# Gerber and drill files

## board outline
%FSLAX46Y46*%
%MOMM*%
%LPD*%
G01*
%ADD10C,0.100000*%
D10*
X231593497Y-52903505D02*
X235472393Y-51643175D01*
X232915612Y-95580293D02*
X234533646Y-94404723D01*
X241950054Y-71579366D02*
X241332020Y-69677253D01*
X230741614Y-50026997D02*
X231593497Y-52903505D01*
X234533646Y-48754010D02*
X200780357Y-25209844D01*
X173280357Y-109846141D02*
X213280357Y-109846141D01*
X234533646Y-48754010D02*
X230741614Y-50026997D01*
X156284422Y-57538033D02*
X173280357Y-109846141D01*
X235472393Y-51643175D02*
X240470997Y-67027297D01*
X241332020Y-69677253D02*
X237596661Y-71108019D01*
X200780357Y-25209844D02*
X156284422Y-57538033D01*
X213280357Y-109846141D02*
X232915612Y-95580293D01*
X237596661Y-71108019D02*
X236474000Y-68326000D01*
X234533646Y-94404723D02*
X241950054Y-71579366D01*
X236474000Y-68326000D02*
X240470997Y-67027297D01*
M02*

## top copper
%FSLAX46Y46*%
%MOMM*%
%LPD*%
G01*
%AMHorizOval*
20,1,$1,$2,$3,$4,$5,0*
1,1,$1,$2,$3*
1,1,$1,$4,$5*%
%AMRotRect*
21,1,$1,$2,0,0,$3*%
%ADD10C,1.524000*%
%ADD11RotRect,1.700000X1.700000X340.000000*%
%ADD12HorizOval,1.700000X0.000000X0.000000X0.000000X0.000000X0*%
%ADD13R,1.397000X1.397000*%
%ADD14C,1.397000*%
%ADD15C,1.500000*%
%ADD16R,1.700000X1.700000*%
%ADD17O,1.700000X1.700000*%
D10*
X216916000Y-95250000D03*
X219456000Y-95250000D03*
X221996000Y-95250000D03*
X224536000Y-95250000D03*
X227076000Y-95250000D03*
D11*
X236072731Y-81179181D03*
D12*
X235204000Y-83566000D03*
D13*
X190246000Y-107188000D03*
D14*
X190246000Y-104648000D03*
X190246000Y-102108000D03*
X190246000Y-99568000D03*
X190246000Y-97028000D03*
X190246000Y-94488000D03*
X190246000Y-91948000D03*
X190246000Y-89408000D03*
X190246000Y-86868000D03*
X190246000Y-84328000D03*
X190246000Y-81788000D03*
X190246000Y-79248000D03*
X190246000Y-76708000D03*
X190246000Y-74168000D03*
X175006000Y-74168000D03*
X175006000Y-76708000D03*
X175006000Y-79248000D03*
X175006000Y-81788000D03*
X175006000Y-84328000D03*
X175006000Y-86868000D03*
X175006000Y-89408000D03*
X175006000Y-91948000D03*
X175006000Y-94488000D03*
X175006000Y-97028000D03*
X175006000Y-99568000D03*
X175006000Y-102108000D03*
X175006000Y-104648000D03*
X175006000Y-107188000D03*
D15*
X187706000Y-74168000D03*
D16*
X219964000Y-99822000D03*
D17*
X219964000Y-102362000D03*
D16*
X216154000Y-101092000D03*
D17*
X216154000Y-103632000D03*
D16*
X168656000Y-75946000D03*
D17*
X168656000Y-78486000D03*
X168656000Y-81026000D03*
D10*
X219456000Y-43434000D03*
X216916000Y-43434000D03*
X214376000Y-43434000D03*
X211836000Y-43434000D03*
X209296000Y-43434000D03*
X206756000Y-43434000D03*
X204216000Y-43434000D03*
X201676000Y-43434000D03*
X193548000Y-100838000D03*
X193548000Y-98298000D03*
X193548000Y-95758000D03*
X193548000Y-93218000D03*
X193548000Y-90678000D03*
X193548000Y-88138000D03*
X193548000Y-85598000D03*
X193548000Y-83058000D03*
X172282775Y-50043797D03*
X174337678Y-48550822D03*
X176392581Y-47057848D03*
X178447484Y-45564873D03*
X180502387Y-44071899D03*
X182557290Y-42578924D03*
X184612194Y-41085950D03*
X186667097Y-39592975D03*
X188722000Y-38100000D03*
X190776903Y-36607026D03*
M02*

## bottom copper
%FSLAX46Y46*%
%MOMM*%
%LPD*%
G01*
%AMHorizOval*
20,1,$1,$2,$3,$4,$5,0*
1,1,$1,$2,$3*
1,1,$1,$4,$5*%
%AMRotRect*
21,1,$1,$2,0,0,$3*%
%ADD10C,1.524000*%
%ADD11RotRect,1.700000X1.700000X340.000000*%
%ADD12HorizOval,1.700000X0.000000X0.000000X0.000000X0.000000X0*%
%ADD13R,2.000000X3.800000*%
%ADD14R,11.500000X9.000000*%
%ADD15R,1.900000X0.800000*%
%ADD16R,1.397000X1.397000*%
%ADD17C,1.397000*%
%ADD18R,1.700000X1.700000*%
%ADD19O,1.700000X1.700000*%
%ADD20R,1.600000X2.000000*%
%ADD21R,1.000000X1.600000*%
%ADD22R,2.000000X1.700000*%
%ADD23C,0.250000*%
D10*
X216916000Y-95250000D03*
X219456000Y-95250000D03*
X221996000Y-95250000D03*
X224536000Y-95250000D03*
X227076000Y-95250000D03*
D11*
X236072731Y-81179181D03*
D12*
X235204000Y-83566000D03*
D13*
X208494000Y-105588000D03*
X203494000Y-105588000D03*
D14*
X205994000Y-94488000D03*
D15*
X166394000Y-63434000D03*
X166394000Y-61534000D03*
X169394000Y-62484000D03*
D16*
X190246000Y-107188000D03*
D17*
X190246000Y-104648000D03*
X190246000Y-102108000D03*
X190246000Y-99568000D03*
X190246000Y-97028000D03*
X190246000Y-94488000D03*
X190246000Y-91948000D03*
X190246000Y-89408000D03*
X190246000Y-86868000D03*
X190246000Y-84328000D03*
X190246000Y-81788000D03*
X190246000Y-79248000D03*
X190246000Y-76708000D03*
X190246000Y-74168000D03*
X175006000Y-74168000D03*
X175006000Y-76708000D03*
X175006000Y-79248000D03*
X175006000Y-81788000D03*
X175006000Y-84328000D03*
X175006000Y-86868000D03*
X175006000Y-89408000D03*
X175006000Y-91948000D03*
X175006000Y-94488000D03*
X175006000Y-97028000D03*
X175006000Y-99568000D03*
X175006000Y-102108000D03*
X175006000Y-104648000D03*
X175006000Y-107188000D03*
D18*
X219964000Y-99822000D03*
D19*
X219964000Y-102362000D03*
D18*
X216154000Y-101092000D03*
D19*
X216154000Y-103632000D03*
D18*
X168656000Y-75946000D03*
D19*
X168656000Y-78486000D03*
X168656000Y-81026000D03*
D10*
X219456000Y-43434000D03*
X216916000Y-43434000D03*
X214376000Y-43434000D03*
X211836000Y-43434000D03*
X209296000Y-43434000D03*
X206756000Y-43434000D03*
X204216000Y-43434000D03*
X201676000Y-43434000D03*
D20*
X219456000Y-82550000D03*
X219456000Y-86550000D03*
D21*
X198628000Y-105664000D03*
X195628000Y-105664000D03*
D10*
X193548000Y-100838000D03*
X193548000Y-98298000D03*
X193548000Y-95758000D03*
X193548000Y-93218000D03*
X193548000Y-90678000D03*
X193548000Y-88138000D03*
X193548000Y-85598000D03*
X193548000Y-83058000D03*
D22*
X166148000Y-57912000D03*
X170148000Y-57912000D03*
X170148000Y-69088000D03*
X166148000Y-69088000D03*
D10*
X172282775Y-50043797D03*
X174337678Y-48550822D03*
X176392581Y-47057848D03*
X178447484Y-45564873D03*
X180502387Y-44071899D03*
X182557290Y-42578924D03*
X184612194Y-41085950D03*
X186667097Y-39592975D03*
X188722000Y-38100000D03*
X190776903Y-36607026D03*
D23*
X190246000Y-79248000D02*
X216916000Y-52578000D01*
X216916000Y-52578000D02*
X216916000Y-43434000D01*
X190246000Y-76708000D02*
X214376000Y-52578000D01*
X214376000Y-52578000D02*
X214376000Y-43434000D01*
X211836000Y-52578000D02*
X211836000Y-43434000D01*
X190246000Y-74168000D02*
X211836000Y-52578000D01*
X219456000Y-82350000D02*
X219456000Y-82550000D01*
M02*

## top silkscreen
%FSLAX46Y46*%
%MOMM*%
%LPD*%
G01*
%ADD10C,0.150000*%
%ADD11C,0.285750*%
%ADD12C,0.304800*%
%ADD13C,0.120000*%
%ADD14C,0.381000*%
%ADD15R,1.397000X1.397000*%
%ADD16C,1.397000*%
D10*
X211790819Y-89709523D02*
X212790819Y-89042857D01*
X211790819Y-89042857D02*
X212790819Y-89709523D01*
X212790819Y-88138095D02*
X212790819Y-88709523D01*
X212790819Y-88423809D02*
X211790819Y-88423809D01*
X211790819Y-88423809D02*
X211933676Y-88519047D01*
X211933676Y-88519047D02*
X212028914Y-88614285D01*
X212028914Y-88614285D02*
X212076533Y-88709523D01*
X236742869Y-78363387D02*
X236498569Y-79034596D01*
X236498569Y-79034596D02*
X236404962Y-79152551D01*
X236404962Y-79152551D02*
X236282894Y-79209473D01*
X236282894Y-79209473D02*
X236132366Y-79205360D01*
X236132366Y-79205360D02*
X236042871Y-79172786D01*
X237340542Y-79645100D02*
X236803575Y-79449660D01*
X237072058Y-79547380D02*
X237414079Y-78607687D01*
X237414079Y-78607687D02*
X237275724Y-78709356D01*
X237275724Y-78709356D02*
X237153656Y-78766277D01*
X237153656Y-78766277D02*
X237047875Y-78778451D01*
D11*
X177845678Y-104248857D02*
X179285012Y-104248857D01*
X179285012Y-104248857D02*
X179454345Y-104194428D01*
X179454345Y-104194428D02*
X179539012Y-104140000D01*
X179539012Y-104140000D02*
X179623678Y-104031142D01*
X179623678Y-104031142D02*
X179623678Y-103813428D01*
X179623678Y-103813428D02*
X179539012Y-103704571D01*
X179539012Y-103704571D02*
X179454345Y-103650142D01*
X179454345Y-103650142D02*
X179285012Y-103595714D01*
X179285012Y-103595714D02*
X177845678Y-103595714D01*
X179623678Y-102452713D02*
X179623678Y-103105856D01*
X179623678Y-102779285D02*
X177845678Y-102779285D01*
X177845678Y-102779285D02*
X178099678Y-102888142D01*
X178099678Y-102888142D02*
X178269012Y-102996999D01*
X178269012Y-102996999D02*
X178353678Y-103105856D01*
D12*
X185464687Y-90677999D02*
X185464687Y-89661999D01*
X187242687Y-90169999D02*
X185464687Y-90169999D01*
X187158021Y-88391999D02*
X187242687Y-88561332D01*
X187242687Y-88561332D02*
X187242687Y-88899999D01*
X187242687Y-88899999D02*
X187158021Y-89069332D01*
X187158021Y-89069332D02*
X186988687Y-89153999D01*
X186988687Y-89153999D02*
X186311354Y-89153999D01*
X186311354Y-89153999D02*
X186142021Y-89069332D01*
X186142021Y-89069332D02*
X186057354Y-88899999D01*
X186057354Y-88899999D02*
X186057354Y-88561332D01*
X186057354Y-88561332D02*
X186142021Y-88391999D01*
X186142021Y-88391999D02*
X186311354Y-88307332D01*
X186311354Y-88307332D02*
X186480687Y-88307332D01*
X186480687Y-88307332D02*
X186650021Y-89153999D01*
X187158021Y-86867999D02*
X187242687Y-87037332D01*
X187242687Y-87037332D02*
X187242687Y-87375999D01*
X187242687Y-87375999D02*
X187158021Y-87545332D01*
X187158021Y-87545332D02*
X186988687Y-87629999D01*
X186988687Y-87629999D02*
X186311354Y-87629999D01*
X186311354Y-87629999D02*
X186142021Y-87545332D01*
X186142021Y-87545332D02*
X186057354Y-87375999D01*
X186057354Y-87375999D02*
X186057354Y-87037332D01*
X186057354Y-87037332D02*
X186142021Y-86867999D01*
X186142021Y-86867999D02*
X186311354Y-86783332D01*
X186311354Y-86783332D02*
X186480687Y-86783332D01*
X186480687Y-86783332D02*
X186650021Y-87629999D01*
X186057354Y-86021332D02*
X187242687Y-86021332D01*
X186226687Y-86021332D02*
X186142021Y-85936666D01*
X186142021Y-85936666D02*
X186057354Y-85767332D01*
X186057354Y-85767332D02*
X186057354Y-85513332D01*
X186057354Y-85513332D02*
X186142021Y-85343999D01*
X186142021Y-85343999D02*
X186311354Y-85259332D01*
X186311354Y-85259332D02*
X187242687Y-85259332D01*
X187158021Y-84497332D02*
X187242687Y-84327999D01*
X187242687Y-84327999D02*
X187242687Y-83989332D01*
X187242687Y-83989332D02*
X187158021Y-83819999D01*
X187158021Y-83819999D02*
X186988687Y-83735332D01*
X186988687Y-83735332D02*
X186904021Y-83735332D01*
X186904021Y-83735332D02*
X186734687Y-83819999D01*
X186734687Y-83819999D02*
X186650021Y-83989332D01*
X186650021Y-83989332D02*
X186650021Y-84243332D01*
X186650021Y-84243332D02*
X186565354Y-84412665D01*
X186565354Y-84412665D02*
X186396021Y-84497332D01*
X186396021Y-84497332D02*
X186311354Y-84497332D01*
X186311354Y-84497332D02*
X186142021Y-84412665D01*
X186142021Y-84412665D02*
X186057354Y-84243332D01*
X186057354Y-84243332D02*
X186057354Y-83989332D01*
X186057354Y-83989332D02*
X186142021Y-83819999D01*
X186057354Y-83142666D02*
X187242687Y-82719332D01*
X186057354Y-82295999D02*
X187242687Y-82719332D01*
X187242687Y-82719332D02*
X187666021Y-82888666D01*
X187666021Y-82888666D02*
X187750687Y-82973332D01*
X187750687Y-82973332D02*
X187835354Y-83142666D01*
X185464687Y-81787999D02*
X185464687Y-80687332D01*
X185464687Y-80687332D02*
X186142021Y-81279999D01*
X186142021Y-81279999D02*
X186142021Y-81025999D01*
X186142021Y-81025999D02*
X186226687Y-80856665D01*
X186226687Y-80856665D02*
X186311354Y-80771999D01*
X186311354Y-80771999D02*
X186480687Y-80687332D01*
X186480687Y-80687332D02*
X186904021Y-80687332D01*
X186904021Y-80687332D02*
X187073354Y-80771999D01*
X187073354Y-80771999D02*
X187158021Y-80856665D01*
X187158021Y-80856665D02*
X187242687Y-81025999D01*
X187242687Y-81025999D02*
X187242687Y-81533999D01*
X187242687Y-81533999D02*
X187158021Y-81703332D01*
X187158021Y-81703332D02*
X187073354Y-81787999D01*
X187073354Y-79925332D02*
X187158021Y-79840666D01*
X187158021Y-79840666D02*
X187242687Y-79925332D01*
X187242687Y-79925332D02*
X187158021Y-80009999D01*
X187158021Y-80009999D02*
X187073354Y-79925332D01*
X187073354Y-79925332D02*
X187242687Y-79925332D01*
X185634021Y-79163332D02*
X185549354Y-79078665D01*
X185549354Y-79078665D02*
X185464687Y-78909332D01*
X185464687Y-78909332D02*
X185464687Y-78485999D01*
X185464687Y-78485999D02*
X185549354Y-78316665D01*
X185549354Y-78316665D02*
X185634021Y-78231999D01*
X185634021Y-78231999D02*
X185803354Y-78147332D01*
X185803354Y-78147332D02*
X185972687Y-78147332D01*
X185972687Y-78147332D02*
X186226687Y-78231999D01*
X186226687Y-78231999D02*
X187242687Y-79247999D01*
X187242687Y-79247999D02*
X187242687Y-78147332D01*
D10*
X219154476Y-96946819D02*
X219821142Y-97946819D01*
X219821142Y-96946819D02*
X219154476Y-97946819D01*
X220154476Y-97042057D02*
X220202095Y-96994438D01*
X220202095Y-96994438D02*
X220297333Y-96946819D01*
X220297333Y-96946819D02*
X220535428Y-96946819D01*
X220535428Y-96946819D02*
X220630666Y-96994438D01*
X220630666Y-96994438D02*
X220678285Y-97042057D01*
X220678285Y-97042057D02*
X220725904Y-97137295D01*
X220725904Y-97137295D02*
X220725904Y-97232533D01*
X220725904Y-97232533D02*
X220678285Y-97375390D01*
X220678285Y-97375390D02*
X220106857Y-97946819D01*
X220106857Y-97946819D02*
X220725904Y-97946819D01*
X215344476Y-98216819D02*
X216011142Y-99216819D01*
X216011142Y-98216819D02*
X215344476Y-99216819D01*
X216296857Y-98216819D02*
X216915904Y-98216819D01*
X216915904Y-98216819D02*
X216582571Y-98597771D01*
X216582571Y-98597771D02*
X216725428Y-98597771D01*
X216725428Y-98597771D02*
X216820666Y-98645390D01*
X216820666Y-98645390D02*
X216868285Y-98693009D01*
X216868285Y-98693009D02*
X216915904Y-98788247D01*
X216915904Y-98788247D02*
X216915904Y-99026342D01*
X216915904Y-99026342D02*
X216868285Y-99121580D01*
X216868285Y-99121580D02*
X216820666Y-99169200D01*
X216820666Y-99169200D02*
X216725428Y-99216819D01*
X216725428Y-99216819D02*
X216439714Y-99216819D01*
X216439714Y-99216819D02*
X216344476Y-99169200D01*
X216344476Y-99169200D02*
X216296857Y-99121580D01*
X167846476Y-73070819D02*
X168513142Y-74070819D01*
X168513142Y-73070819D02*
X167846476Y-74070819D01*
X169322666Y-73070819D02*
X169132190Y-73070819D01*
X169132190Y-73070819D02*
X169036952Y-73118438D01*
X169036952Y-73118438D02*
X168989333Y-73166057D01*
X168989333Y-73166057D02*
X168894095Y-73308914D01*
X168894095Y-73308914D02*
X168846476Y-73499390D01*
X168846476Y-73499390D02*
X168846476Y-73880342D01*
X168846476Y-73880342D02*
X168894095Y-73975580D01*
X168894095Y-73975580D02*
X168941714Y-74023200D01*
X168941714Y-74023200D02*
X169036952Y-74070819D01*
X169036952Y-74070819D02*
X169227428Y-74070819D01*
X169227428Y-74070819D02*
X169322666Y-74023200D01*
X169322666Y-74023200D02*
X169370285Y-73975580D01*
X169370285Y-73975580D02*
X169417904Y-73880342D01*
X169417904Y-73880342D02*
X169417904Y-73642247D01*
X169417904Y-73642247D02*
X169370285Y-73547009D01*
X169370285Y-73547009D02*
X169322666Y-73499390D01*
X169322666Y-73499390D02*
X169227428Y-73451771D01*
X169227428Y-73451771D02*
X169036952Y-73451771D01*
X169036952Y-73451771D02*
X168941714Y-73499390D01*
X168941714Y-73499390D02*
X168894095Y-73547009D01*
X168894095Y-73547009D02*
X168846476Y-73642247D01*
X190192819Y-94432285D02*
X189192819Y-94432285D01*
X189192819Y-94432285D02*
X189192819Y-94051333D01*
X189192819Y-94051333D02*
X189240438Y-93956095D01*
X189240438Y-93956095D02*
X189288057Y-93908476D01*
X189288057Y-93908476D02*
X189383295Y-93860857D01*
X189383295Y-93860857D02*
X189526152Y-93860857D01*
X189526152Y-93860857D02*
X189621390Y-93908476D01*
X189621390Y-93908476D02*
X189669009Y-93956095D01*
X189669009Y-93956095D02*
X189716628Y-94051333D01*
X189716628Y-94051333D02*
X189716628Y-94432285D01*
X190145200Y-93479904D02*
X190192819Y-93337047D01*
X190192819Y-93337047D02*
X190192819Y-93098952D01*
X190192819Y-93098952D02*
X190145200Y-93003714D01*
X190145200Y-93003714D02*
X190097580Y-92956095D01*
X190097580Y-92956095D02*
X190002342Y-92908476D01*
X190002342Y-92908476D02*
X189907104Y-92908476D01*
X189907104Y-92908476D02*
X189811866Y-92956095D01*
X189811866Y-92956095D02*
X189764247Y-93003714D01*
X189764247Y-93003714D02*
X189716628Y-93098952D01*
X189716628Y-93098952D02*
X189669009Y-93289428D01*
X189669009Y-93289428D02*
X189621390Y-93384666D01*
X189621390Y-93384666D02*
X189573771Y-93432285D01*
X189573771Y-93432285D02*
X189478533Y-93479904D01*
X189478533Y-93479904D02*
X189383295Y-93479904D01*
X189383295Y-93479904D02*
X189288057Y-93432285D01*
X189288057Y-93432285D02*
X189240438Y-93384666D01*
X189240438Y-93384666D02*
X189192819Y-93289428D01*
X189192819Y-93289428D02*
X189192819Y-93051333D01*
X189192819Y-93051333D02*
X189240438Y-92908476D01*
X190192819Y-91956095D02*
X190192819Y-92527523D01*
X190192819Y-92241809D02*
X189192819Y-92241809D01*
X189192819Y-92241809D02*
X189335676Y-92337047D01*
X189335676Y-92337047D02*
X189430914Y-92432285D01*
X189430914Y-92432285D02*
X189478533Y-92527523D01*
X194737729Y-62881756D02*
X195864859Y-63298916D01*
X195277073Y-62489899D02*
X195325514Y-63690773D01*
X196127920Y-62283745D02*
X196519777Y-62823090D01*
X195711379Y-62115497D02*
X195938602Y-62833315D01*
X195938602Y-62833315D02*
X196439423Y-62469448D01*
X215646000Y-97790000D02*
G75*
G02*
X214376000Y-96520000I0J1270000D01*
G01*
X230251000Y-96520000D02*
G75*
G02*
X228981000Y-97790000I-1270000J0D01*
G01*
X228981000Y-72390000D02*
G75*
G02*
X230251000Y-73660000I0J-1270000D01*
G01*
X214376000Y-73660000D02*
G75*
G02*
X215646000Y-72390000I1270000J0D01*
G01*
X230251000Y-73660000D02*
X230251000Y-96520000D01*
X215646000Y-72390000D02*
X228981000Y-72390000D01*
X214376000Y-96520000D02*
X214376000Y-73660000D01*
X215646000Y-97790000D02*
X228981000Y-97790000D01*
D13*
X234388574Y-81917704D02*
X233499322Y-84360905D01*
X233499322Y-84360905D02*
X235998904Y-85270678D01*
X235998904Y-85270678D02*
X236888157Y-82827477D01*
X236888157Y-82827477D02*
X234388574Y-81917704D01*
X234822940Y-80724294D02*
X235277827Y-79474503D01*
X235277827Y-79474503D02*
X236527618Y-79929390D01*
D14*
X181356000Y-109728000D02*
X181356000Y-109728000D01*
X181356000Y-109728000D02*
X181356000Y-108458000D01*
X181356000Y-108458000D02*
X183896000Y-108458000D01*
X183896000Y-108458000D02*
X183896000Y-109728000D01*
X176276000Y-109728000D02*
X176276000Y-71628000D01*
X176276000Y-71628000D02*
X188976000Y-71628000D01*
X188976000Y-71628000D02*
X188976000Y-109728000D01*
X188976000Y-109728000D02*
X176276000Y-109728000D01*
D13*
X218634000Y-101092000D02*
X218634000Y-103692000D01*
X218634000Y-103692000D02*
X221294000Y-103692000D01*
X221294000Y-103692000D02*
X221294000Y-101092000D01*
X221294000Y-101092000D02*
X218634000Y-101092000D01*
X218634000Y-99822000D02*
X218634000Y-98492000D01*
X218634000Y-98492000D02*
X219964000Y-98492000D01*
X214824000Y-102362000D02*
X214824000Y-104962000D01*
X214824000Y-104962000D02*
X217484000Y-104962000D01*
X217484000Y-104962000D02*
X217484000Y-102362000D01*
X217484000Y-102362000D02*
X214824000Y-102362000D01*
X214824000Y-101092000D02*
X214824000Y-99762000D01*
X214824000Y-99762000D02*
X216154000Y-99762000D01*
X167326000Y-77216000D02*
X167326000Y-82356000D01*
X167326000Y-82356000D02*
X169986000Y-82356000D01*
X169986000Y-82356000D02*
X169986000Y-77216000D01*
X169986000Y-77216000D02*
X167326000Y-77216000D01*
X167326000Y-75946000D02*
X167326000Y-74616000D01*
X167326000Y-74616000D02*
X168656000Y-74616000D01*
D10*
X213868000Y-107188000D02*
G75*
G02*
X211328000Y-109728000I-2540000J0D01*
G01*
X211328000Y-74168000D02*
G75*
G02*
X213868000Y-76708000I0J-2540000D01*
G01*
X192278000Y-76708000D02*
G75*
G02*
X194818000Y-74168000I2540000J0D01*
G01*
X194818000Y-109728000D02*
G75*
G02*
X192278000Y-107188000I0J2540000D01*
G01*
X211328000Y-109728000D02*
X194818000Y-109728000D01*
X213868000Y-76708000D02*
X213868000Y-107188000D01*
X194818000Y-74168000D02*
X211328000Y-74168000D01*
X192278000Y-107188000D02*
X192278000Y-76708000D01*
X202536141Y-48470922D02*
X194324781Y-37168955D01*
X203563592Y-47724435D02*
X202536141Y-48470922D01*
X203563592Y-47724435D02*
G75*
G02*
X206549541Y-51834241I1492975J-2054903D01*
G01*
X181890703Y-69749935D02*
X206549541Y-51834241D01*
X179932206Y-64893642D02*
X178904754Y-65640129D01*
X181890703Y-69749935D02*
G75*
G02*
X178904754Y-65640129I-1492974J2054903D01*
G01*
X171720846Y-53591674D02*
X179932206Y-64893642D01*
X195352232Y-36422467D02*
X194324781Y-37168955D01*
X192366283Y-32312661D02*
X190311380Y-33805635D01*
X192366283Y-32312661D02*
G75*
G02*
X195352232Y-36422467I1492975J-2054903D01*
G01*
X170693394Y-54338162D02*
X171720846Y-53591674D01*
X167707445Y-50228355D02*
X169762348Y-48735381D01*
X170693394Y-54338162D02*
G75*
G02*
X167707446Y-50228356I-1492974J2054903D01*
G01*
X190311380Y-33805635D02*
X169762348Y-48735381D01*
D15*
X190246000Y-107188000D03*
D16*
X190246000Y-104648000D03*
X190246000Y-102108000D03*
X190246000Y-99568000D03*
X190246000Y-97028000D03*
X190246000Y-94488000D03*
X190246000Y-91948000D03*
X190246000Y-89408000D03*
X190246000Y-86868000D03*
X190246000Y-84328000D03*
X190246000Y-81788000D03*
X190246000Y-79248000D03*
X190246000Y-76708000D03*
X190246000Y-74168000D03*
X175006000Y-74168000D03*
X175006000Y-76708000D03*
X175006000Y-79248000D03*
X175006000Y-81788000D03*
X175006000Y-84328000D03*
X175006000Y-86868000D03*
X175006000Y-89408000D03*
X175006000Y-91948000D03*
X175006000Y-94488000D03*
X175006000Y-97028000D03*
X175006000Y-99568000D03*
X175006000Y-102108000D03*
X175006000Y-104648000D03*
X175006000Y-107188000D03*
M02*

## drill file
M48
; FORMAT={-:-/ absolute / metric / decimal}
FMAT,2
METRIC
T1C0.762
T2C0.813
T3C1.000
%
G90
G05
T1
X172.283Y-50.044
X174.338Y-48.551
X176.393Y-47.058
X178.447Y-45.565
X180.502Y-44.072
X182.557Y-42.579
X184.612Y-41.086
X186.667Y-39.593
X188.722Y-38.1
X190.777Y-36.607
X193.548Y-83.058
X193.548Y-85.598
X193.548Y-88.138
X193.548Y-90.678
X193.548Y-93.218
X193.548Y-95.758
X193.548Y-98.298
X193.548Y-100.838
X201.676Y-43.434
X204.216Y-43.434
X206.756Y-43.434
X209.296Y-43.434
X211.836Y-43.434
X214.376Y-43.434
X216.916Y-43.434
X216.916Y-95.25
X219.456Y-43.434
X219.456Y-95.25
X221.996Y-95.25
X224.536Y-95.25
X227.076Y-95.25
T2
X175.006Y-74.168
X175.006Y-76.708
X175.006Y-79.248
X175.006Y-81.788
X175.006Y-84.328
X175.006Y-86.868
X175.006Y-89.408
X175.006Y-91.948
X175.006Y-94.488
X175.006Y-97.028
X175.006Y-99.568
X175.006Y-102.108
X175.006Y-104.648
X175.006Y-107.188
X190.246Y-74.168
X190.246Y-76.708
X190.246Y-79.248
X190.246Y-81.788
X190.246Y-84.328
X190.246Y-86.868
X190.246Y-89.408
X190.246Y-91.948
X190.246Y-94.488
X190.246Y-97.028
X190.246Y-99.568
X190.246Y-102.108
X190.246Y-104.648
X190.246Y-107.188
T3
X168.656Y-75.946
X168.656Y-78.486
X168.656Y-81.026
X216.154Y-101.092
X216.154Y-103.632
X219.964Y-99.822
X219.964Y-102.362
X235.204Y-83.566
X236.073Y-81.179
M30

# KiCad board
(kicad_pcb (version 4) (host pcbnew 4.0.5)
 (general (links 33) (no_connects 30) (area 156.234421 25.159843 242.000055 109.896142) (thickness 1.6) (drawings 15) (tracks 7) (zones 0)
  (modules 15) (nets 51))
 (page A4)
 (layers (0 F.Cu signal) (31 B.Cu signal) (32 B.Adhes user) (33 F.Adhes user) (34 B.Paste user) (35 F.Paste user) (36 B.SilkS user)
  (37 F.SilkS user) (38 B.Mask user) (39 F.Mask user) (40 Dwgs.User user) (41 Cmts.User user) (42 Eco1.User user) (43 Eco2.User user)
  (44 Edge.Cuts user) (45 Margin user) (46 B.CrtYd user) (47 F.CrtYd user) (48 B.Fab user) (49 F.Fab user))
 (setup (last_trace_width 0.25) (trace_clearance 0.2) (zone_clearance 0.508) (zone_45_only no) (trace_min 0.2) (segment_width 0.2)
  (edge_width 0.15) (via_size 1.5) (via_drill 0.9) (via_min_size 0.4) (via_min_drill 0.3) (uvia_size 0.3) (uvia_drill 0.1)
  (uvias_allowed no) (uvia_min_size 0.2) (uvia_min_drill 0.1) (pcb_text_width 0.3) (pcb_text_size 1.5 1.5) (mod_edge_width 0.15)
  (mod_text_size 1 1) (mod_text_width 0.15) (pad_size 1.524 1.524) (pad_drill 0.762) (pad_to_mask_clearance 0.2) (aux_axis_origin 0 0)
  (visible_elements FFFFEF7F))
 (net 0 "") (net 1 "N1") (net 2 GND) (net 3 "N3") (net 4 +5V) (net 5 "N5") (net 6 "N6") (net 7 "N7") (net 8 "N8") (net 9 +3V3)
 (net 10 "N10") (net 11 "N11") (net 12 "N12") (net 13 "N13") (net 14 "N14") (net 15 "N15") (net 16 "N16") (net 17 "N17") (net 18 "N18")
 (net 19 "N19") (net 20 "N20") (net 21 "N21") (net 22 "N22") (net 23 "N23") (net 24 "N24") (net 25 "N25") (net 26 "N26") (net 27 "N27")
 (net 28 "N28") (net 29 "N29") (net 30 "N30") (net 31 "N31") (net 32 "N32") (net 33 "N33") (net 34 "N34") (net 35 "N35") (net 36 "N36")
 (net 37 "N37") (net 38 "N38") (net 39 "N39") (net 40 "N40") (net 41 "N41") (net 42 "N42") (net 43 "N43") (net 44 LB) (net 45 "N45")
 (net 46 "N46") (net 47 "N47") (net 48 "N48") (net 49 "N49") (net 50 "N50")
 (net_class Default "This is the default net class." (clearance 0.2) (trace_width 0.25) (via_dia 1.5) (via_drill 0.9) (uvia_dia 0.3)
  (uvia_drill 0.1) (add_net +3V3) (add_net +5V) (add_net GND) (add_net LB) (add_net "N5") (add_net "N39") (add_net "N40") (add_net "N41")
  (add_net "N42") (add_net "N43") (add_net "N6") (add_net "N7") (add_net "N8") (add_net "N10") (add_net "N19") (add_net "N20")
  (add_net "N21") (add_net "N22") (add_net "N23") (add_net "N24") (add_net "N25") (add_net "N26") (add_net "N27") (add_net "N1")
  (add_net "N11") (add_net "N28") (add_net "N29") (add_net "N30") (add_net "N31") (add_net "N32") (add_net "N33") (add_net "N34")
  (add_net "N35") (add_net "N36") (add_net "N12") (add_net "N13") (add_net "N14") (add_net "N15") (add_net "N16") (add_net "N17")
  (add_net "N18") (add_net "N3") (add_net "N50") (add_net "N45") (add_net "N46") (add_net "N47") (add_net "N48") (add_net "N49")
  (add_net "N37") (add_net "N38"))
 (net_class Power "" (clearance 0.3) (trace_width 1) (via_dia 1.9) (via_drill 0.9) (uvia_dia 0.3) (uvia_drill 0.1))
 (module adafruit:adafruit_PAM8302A (layer F.Cu) (at 219.456 88.9 90)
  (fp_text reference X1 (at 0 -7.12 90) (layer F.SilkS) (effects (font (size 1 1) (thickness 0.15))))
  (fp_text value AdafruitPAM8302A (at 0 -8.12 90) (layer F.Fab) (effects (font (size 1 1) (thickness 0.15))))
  (fp_arc (start -7.62 -3.81) (end -8.89 -3.81) (angle 90) (layer F.SilkS) (width 0.15))
  (fp_arc (start -7.62 9.525) (end -7.62 10.795) (angle 90) (layer F.SilkS) (width 0.15))
  (fp_arc (start 15.24 9.525) (end 16.51 9.525) (angle 90) (layer F.SilkS) (width 0.15))
  (fp_arc (start 15.24 -3.81) (end 15.24 -5.08) (angle 90) (layer F.SilkS) (width 0.15))
  (fp_line (start 15.24 10.795) (end -7.62 10.795) (layer F.SilkS) (width 0.15))
  (fp_line (start 16.51 -3.81) (end 16.51 9.525) (layer F.SilkS) (width 0.15))
  (fp_line (start -7.62 -5.08) (end 15.24 -5.08) (layer F.SilkS) (width 0.15))
  (fp_line (start -8.89 -3.81) (end -8.89 9.525) (layer F.SilkS) (width 0.15))
  (pad 1 thru_hole circle (at -6.35 -2.54 90) (size 1.524 1.524) (drill 0.762) (layers *.Cu *.Mask) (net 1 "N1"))
  (pad 2 thru_hole circle (at -6.35 0 90) (size 1.524 1.524) (drill 0.762) (layers *.Cu *.Mask) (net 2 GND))
  (pad 3 thru_hole circle (at -6.35 2.54 90) (size 1.524 1.524) (drill 0.762) (layers *.Cu *.Mask) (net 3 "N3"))
  (pad 4 thru_hole circle (at -6.35 5.08 90) (size 1.524 1.524) (drill 0.762) (layers *.Cu *.Mask) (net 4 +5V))
  (pad 5 thru_hole circle (at -6.35 7.62 90) (size 1.524 1.524) (drill 0.762) (layers *.Cu *.Mask) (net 2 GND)))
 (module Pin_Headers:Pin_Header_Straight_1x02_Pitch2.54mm (layer F.Cu) (at 236.072731 81.179181 340)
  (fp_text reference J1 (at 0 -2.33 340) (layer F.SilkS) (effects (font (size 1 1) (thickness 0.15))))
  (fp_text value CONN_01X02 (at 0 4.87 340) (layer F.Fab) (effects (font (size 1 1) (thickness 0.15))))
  (fp_line (start -1.33 1.27) (end -1.33 3.87) (layer F.SilkS) (width 0.12))
  (fp_line (start -1.33 3.87) (end 1.33 3.87) (layer F.SilkS) (width 0.12))
  (fp_line (start 1.33 3.87) (end 1.33 1.27) (layer F.SilkS) (width 0.12))
  (fp_line (start 1.33 1.27) (end -1.33 1.27) (layer F.SilkS) (width 0.12))
  (fp_line (start -1.33 0) (end -1.33 -1.33) (layer F.SilkS) (width 0.12))
  (fp_line (start -1.33 -1.33) (end 0 -1.33) (layer F.SilkS) (width 0.12))
  (pad 1 thru_hole rect (at 0 0 340) (size 1.7 1.7) (drill 1) (layers *.Cu *.Mask) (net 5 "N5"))
  (pad 2 thru_hole oval (at 0 2.54 340) (size 1.7 1.7) (drill 1) (layers *.Cu *.Mask) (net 2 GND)))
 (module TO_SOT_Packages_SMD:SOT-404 (layer B.Cu) (at 205.994 100.038 90)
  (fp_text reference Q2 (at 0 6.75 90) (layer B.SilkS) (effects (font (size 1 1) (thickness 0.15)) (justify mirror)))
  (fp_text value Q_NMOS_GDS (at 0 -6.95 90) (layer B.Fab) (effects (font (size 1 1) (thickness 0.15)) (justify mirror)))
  (pad 1 smd rect (at -5.55 2.5 180) (size 2 3.8) (layers B.Cu B.Paste B.Mask) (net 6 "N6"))
  (pad 3 smd rect (at -5.55 -2.5 180) (size 2 3.8) (layers B.Cu B.Paste B.Mask) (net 2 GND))
  (pad 2 smd rect (at 5.55 0 180) (size 11.5 9) (layers B.Cu B.Paste B.Mask) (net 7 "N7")))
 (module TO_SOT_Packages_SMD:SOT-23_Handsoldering (layer B.Cu) (at 167.894 62.484)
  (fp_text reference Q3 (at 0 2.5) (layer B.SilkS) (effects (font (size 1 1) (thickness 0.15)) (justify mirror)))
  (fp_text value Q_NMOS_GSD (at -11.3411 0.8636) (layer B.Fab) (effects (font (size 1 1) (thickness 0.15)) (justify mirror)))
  (pad 1 smd rect (at -1.5 0.95) (size 1.9 0.8) (layers B.Cu B.Paste B.Mask) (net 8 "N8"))
  (pad 2 smd rect (at -1.5 -0.95) (size 1.9 0.8) (layers B.Cu B.Paste B.Mask) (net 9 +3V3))
  (pad 3 smd rect (at 1.5 0) (size 1.9 0.8) (layers B.Cu B.Paste B.Mask) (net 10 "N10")))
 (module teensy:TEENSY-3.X (layer F.Cu) (at 182.626 90.678 90)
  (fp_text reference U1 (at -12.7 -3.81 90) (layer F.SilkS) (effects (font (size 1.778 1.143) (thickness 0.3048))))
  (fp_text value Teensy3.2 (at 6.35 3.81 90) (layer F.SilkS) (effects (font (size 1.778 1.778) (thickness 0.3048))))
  (fp_line (start -19.05 -1.27) (end -19.05 -1.27) (layer F.SilkS) (width 0.381))
  (fp_line (start -19.05 -1.27) (end -17.78 -1.27) (layer F.SilkS) (width 0.381))
  (fp_line (start -17.78 -1.27) (end -17.78 1.27) (layer F.SilkS) (width 0.381))
  (fp_line (start -17.78 1.27) (end -19.05 1.27) (layer F.SilkS) (width 0.381))
  (fp_line (start -19.05 -6.35) (end 19.05 -6.35) (layer F.SilkS) (width 0.381))
  (fp_line (start 19.05 -6.35) (end 19.05 6.35) (layer F.SilkS) (width 0.381))
  (fp_line (start 19.05 6.35) (end -19.05 6.35) (layer F.SilkS) (width 0.381))
  (fp_line (start -19.05 6.35) (end -19.05 -6.35) (layer F.SilkS) (width 0.381))
  (pad 1 thru_hole rect (at -16.51 7.62 90) (size 1.397 1.397) (drill 0.8128) (layers *.Cu *.Mask F.SilkS) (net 2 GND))
  (pad 2 thru_hole circle (at -13.97 7.62 90) (size 1.397 1.397) (drill 0.8128) (layers *.Cu *.Mask F.SilkS) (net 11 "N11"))
  (pad 3 thru_hole circle (at -11.43 7.62 90) (size 1.397 1.397) (drill 0.8128) (layers *.Cu *.Mask F.SilkS) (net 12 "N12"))
  (pad 4 thru_hole circle (at -8.89 7.62 90) (size 1.397 1.397) (drill 0.8128) (layers *.Cu *.Mask F.SilkS) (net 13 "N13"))
  (pad 5 thru_hole circle (at -6.35 7.62 90) (size 1.397 1.397) (drill 0.8128) (layers *.Cu *.Mask F.SilkS) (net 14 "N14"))
  (pad 6 thru_hole circle (at -3.81 7.62 90) (size 1.397 1.397) (drill 0.8128) (layers *.Cu *.Mask F.SilkS) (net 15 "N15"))
  (pad 7 thru_hole circle (at -1.27 7.62 90) (size 1.397 1.397) (drill 0.8128) (layers *.Cu *.Mask F.SilkS) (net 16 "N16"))
  (pad 8 thru_hole circle (at 1.27 7.62 90) (size 1.397 1.397) (drill 0.8128) (layers *.Cu *.Mask F.SilkS) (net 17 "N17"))
  (pad 9 thru_hole circle (at 3.81 7.62 90) (size 1.397 1.397) (drill 0.8128) (layers *.Cu *.Mask F.SilkS) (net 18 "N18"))
  (pad 10 thru_hole circle (at 6.35 7.62 90) (size 1.397 1.397) (drill 0.8128) (layers *.Cu *.Mask F.SilkS) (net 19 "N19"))
  (pad 11 thru_hole circle (at 8.89 7.62 90) (size 1.397 1.397) (drill 0.8128) (layers *.Cu *.Mask F.SilkS) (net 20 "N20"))
  (pad 12 thru_hole circle (at 11.43 7.62 90) (size 1.397 1.397) (drill 0.8128) (layers *.Cu *.Mask F.SilkS) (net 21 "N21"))
  (pad 13 thru_hole circle (at 13.97 7.62 90) (size 1.397 1.397) (drill 0.8128) (layers *.Cu *.Mask F.SilkS) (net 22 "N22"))
  (pad 14 thru_hole circle (at 16.51 7.62 90) (size 1.397 1.397) (drill 0.8128) (layers *.Cu *.Mask F.SilkS) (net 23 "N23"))
  (pad 15 thru_hole circle (at 16.51 -7.62 90) (size 1.397 1.397) (drill 0.8128) (layers *.Cu *.Mask F.SilkS) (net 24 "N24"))
  (pad 16 thru_hole circle (at 13.97 -7.62 90) (size 1.397 1.397) (drill 0.8128) (layers *.Cu *.Mask F.SilkS) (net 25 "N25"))
  (pad 17 thru_hole circle (at 11.43 -7.62 90) (size 1.397 1.397) (drill 0.8128) (layers *.Cu *.Mask F.SilkS) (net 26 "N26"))
  (pad 18 thru_hole circle (at 8.89 -7.62 90) (size 1.397 1.397) (drill 0.8128) (layers *.Cu *.Mask F.SilkS) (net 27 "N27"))
  (pad 19 thru_hole circle (at 6.35 -7.62 90) (size 1.397 1.397) (drill 0.8128) (layers *.Cu *.Mask F.SilkS) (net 1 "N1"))
  (pad 20 thru_hole circle (at 3.81 -7.62 90) (size 1.397 1.397) (drill 0.8128) (layers *.Cu *.Mask F.SilkS) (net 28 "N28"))
  (pad 21 thru_hole circle (at 1.27 -7.62 90) (size 1.397 1.397) (drill 0.8128) (layers *.Cu *.Mask F.SilkS) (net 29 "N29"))
  (pad 22 thru_hole circle (at -1.27 -7.62 90) (size 1.397 1.397) (drill 0.8128) (layers *.Cu *.Mask F.SilkS) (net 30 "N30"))
  (pad 23 thru_hole circle (at -3.81 -7.62 90) (size 1.397 1.397) (drill 0.8128) (layers *.Cu *.Mask F.SilkS) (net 7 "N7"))
  (pad 24 thru_hole circle (at -6.35 -7.62 90) (size 1.397 1.397) (drill 0.8128) (layers *.Cu *.Mask F.SilkS) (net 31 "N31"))
  (pad 25 thru_hole circle (at -8.89 -7.62 90) (size 1.397 1.397) (drill 0.8128) (layers *.Cu *.Mask F.SilkS) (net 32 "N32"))
  (pad 26 thru_hole circle (at -11.43 -7.62 90) (size 1.397 1.397) (drill 0.8128) (layers *.Cu *.Mask F.SilkS) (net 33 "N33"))
  (pad 27 thru_hole circle (at -13.97 -7.62 90) (size 1.397 1.397) (drill 0.8128) (layers *.Cu *.Mask F.SilkS) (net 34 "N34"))
  (pad 28 thru_hole circle (at -16.51 -7.62 90) (size 1.397 1.397) (drill 0.8128) (layers *.Cu *.Mask F.SilkS) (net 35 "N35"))
  (pad 29 smd circle (at 16.51 5.08 90) (size 1.5 1.5) (layers F.Cu F.Paste F.Mask) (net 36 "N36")))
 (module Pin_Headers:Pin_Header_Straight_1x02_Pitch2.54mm (layer F.Cu) (at 219.964 99.822)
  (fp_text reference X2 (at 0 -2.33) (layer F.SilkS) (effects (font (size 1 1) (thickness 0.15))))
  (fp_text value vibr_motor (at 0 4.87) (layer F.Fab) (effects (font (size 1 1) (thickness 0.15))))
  (fp_line (start -1.33 1.27) (end -1.33 3.87) (layer F.SilkS) (width 0.12))
  (fp_line (start -1.33 3.87) (end 1.33 3.87) (layer F.SilkS) (width 0.12))
  (fp_line (start 1.33 3.87) (end 1.33 1.27) (layer F.SilkS) (width 0.12))
  (fp_line (start 1.33 1.27) (end -1.33 1.27) (layer F.SilkS) (width 0.12))
  (fp_line (start -1.33 0) (end -1.33 -1.33) (layer F.SilkS) (width 0.12))
  (fp_line (start -1.33 -1.33) (end 0 -1.33) (layer F.SilkS) (width 0.12))
  (pad 1 thru_hole rect (at 0 0) (size 1.7 1.7) (drill 1) (layers *.Cu *.Mask) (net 6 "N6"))
  (pad 2 thru_hole oval (at 0 2.54) (size 1.7 1.7) (drill 1) (layers *.Cu *.Mask) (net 9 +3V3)))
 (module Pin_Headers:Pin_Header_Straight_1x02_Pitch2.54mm (layer F.Cu) (at 216.154 101.092)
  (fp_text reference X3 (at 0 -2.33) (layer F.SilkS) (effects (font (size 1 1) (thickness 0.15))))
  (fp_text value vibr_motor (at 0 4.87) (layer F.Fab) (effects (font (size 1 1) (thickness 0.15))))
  (fp_line (start -1.33 1.27) (end -1.33 3.87) (layer F.SilkS) (width 0.12))
  (fp_line (start -1.33 3.87) (end 1.33 3.87) (layer F.SilkS) (width 0.12))
  (fp_line (start 1.33 3.87) (end 1.33 1.27) (layer F.SilkS) (width 0.12))
  (fp_line (start 1.33 1.27) (end -1.33 1.27) (layer F.SilkS) (width 0.12))
  (fp_line (start -1.33 0) (end -1.33 -1.33) (layer F.SilkS) (width 0.12))
  (fp_line (start -1.33 -1.33) (end 0 -1.33) (layer F.SilkS) (width 0.12))
  (pad 1 thru_hole rect (at 0 0) (size 1.7 1.7) (drill 1) (layers *.Cu *.Mask) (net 6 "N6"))
  (pad 2 thru_hole oval (at 0 2.54) (size 1.7 1.7) (drill 1) (layers *.Cu *.Mask) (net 9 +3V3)))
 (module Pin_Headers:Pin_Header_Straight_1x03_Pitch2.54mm (layer F.Cu) (at 168.656 75.946)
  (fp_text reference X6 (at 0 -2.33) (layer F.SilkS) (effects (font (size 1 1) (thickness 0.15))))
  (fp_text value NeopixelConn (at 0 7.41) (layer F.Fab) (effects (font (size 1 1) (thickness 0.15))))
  (fp_line (start -1.33 1.27) (end -1.33 6.41) (layer F.SilkS) (width 0.12))
  (fp_line (start -1.33 6.41) (end 1.33 6.41) (layer F.SilkS) (width 0.12))
  (fp_line (start 1.33 6.41) (end 1.33 1.27) (layer F.SilkS) (width 0.12))
  (fp_line (start 1.33 1.27) (end -1.33 1.27) (layer F.SilkS) (width 0.12))
  (fp_line (start -1.33 0) (end -1.33 -1.33) (layer F.SilkS) (width 0.12))
  (fp_line (start -1.33 -1.33) (end 0 -1.33) (layer F.SilkS) (width 0.12))
  (pad 1 thru_hole rect (at 0 0) (size 1.7 1.7) (drill 1) (layers *.Cu *.Mask) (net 8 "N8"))
  (pad 2 thru_hole oval (at 0 2.54) (size 1.7 1.7) (drill 1) (layers *.Cu *.Mask) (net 4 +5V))
  (pad 3 thru_hole oval (at 0 5.08) (size 1.7 1.7) (drill 1) (layers *.Cu *.Mask) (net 2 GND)))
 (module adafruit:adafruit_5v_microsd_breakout (layer B.Cu) (at 210.566 52.324 90)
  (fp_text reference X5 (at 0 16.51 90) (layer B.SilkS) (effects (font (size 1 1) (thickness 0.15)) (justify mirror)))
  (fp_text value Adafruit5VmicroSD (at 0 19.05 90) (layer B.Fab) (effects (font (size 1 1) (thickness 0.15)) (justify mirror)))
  (pad 1 thru_hole circle (at 8.89 8.89 90) (size 1.524 1.524) (drill 0.762) (layers *.Cu *.Mask) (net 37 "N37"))
  (pad 2 thru_hole circle (at 8.89 6.35 90) (size 1.524 1.524) (drill 0.762) (layers *.Cu *.Mask) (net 21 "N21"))
  (pad 3 thru_hole circle (at 8.89 3.81 90) (size 1.524 1.524) (drill 0.762) (layers *.Cu *.Mask) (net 22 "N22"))
  (pad 4 thru_hole circle (at 8.89 1.27 90) (size 1.524 1.524) (drill 0.762) (layers *.Cu *.Mask) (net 23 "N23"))
  (pad 5 thru_hole circle (at 8.89 -1.27 90) (size 1.524 1.524) (drill 0.762) (layers *.Cu *.Mask) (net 28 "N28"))
  (pad 6 thru_hole circle (at 8.89 -3.81 90) (size 1.524 1.524) (drill 0.762) (layers *.Cu *.Mask) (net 2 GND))
  (pad 7 thru_hole circle (at 8.89 -6.35 90) (size 1.524 1.524) (drill 0.762) (layers *.Cu *.Mask) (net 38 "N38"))
  (pad 8 thru_hole circle (at 8.89 -8.89 90) (size 1.524 1.524) (drill 0.762) (layers *.Cu *.Mask) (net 4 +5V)))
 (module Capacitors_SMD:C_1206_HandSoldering (layer B.Cu) (at 219.456 84.55 270)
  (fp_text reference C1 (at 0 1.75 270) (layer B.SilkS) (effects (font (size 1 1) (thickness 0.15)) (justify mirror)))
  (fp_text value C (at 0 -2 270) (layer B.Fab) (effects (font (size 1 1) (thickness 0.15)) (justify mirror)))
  (pad 1 smd rect (at -2 0 270) (size 2 1.6) (layers B.Cu B.Paste B.Mask) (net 5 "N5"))
  (pad 2 smd rect (at 2 0 270) (size 2 1.6) (layers B.Cu B.Paste B.Mask) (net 2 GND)))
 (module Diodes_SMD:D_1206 (layer B.Cu) (at 197.128 105.664 180)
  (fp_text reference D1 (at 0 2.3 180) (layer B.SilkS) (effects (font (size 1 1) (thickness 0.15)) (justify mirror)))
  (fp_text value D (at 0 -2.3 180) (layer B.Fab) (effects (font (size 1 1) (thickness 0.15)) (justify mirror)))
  (pad 1 smd rect (at -1.5 0 180) (size 1 1.6) (layers B.Cu B.Paste B.Mask) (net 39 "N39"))
  (pad 2 smd rect (at 1.5 0 180) (size 1 1.6) (layers B.Cu B.Paste B.Mask) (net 2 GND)))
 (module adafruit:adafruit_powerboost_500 (layer F.Cu) (at 202.438 93.218 90)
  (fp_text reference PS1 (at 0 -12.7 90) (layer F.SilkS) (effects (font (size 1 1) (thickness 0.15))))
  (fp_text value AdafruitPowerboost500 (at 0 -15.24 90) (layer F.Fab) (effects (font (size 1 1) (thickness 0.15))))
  (fp_arc (start -13.97 8.89) (end -13.97 11.43) (angle 90) (layer F.SilkS) (width 0.15))
  (fp_arc (start 16.51 8.89) (end 19.05 8.89) (angle 90) (layer F.SilkS) (width 0.15))
  (fp_arc (start 16.51 -7.62) (end 16.51 -10.16) (angle 90) (layer F.SilkS) (width 0.15))
  (fp_arc (start -13.97 -7.62) (end -16.51 -7.62) (angle 90) (layer F.SilkS) (width 0.15))
  (fp_line (start -16.51 8.89) (end -16.51 -7.62) (layer F.SilkS) (width 0.15))
  (fp_line (start 16.51 11.43) (end -13.97 11.43) (layer F.SilkS) (width 0.15))
  (fp_line (start 19.05 -7.62) (end 19.05 8.89) (layer F.SilkS) (width 0.15))
  (fp_line (start -13.97 -10.16) (end 16.51 -10.16) (layer F.SilkS) (width 0.15))
  (pad 1 thru_hole circle (at -7.62 -8.89 90) (size 1.524 1.524) (drill 0.762) (layers *.Cu *.Mask) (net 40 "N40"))
  (pad 2 thru_hole circle (at -5.08 -8.89 90) (size 1.524 1.524) (drill 0.762) (layers *.Cu *.Mask) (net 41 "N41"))
  (pad 3 thru_hole circle (at -2.54 -8.89 90) (size 1.524 1.524) (drill 0.762) (layers *.Cu *.Mask) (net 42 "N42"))
  (pad 4 thru_hole circle (at 0 -8.89 90) (size 1.524 1.524) (drill 0.762) (layers *.Cu *.Mask) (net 5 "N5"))
  (pad 5 thru_hole circle (at 2.54 -8.89 90) (size 1.524 1.524) (drill 0.762) (layers *.Cu *.Mask) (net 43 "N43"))
  (pad 6 thru_hole circle (at 5.08 -8.89 90) (size 1.524 1.524) (drill 0.762) (layers *.Cu *.Mask) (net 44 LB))
  (pad 7 thru_hole circle (at 7.62 -8.89 90) (size 1.524 1.524) (drill 0.762) (layers *.Cu *.Mask) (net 2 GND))
  (pad 8 thru_hole circle (at 10.16 -8.89 90) (size 1.524 1.524) (drill 0.762) (layers *.Cu *.Mask) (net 4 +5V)))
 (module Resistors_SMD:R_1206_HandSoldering (layer B.Cu) (at 168.148 57.912)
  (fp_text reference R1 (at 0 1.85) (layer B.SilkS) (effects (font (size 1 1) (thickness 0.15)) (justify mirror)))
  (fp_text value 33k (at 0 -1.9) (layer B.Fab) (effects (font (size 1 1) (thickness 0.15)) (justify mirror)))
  (pad 1 smd rect (at -2 0) (size 2 1.7) (layers B.Cu B.Paste B.Mask) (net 9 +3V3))
  (pad 2 smd rect (at 2 0) (size 2 1.7) (layers B.Cu B.Paste B.Mask) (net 10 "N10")))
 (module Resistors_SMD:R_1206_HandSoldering (layer B.Cu) (at 168.148 69.088 180)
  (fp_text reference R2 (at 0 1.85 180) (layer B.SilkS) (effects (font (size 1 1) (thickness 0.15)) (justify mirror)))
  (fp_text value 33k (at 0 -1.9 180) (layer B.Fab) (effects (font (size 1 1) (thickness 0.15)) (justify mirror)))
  (pad 1 smd rect (at -2 0 180) (size 2 1.7) (layers B.Cu B.Paste B.Mask) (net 4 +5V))
  (pad 2 smd rect (at 2 0 180) (size 2 1.7) (layers B.Cu B.Paste B.Mask) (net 8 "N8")))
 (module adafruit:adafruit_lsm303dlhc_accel (layer F.Cu) (at 187.501737 51.545024 216)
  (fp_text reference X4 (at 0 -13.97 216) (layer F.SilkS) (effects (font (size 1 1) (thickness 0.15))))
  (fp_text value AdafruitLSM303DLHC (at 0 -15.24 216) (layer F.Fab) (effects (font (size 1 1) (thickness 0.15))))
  (fp_line (start -13.97 -6.35) (end -13.97 7.62) (layer F.SilkS) (width 0.15))
  (fp_line (start -15.24 -6.35) (end -13.97 -6.35) (layer F.SilkS) (width 0.15))
  (fp_arc (start -15.24 -8.89) (end -15.24 -6.35) (angle 180) (layer F.SilkS) (width 0.15))
  (fp_line (start 15.24 -11.43) (end -15.24 -11.43) (layer F.SilkS) (width 0.15))
  (fp_line (start 13.97 -6.35) (end 15.24 -6.35) (layer F.SilkS) (width 0.15))
  (fp_arc (start 15.24 -8.89) (end 15.24 -11.43) (angle 180) (layer F.SilkS) (width 0.15))
  (fp_line (start 13.97 7.62) (end 13.97 -6.35) (layer F.SilkS) (width 0.15))
  (fp_line (start -15.24 7.62) (end -13.97 7.62) (layer F.SilkS) (width 0.15))
  (fp_line (start -15.24 12.7) (end -12.7 12.7) (layer F.SilkS) (width 0.15))
  (fp_arc (start -15.24 10.16) (end -15.24 12.7) (angle 180) (layer F.SilkS) (width 0.15))
  (fp_line (start 15.24 7.62) (end 13.97 7.62) (layer F.SilkS) (width 0.15))
  (fp_line (start 15.24 12.7) (end 12.7 12.7) (layer F.SilkS) (width 0.15))
  (fp_arc (start 15.24 10.16) (end 15.24 7.62) (angle 180) (layer F.SilkS) (width 0.15))
  (fp_line (start -12.7 12.7) (end 12.7 12.7) (layer F.SilkS) (width 0.15))
  (pad 1 thru_hole circle (at 11.43 10.16 216) (size 1.524 1.524) (drill 0.762) (layers *.Cu *.Mask) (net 9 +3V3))
  (pad 2 thru_hole circle (at 8.89 10.16 216) (size 1.524 1.524) (drill 0.762) (layers *.Cu *.Mask) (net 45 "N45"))
  (pad 3 thru_hole circle (at 6.35 10.16 216) (size 1.524 1.524) (drill 0.762) (layers *.Cu *.Mask) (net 2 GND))
  (pad 4 thru_hole circle (at 3.81 10.16 216) (size 1.524 1.524) (drill 0.762) (layers *.Cu *.Mask) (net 33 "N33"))
  (pad 5 thru_hole circle (at 1.27 10.16 216) (size 1.524 1.524) (drill 0.762) (layers *.Cu *.Mask) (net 32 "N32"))
  (pad 6 thru_hole circle (at -1.27 10.16 216) (size 1.524 1.524) (drill 0.762) (layers *.Cu *.Mask) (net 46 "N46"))
  (pad 7 thru_hole circle (at -3.81 10.16 216) (size 1.524 1.524) (drill 0.762) (layers *.Cu *.Mask) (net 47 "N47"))
  (pad 8 thru_hole circle (at -6.35 10.16 216) (size 1.524 1.524) (drill 0.762) (layers *.Cu *.Mask) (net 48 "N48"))
  (pad 9 thru_hole circle (at -8.89 10.16 216) (size 1.524 1.524) (drill 0.762) (layers *.Cu *.Mask) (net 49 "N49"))
  (pad 10 thru_hole circle (at -11.43 10.16 216) (size 1.524 1.524) (drill 0.762) (layers *.Cu *.Mask) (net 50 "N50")))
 (gr_line (start 231.593497 52.903505) (end 235.472393 51.643175) (layer Edge.Cuts) (width 0.1))
 (gr_line (start 232.915612 95.580293) (end 234.533646 94.404723) (layer Edge.Cuts) (width 0.1))
 (gr_line (start 241.950054 71.579366) (end 241.33202 69.677253) (layer Edge.Cuts) (width 0.1))
 (gr_line (start 230.741614 50.026997) (end 231.593497 52.903505) (layer Edge.Cuts) (width 0.1))
 (gr_line (start 234.533646 48.75401) (end 200.780357 25.209844) (layer Edge.Cuts) (width 0.1))
 (gr_line (start 173.280357 109.846141) (end 213.280357 109.846141) (layer Edge.Cuts) (width 0.1))
 (gr_line (start 234.533646 48.75401) (end 230.741614 50.026997) (layer Edge.Cuts) (width 0.1))
 (gr_line (start 156.284422 57.538033) (end 173.280357 109.846141) (layer Edge.Cuts) (width 0.1))
 (gr_line (start 235.472393 51.643175) (end 240.470997 67.027297) (layer Edge.Cuts) (width 0.1))
 (gr_line (start 241.33202 69.677253) (end 237.596661 71.108019) (layer Edge.Cuts) (width 0.1))
 (gr_line (start 200.780357 25.209844) (end 156.284422 57.538033) (layer Edge.Cuts) (width 0.1))
 (gr_line (start 213.280357 109.846141) (end 232.915612 95.580293) (layer Edge.Cuts) (width 0.1))
 (gr_line (start 237.596661 71.108019) (end 236.474 68.326) (layer Edge.Cuts) (width 0.1))
 (gr_line (start 234.533646 94.404723) (end 241.950054 71.579366) (layer Edge.Cuts) (width 0.1))
 (gr_line (start 236.474 68.326) (end 240.470997 67.027297) (layer Edge.Cuts) (width 0.1))
 (segment (start 190.246 79.248) (end 216.916 52.578) (width 0.25) (layer B.Cu) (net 21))
 (segment (start 216.916 52.578) (end 216.916 43.434) (width 0.25) (layer B.Cu) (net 21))
 (segment (start 190.246 76.708) (end 214.376 52.578) (width 0.25) (layer B.Cu) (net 22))
 (segment (start 214.376 52.578) (end 214.376 43.434) (width 0.25) (layer B.Cu) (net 22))
 (segment (start 211.836 52.578) (end 211.836 43.434) (width 0.25) (layer B.Cu) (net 23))
 (segment (start 190.246 74.168) (end 211.836 52.578) (width 0.25) (layer B.Cu) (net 23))
 (segment (start 219.456 82.35) (end 219.456 82.55) (width 0.25) (layer B.Cu) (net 5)))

